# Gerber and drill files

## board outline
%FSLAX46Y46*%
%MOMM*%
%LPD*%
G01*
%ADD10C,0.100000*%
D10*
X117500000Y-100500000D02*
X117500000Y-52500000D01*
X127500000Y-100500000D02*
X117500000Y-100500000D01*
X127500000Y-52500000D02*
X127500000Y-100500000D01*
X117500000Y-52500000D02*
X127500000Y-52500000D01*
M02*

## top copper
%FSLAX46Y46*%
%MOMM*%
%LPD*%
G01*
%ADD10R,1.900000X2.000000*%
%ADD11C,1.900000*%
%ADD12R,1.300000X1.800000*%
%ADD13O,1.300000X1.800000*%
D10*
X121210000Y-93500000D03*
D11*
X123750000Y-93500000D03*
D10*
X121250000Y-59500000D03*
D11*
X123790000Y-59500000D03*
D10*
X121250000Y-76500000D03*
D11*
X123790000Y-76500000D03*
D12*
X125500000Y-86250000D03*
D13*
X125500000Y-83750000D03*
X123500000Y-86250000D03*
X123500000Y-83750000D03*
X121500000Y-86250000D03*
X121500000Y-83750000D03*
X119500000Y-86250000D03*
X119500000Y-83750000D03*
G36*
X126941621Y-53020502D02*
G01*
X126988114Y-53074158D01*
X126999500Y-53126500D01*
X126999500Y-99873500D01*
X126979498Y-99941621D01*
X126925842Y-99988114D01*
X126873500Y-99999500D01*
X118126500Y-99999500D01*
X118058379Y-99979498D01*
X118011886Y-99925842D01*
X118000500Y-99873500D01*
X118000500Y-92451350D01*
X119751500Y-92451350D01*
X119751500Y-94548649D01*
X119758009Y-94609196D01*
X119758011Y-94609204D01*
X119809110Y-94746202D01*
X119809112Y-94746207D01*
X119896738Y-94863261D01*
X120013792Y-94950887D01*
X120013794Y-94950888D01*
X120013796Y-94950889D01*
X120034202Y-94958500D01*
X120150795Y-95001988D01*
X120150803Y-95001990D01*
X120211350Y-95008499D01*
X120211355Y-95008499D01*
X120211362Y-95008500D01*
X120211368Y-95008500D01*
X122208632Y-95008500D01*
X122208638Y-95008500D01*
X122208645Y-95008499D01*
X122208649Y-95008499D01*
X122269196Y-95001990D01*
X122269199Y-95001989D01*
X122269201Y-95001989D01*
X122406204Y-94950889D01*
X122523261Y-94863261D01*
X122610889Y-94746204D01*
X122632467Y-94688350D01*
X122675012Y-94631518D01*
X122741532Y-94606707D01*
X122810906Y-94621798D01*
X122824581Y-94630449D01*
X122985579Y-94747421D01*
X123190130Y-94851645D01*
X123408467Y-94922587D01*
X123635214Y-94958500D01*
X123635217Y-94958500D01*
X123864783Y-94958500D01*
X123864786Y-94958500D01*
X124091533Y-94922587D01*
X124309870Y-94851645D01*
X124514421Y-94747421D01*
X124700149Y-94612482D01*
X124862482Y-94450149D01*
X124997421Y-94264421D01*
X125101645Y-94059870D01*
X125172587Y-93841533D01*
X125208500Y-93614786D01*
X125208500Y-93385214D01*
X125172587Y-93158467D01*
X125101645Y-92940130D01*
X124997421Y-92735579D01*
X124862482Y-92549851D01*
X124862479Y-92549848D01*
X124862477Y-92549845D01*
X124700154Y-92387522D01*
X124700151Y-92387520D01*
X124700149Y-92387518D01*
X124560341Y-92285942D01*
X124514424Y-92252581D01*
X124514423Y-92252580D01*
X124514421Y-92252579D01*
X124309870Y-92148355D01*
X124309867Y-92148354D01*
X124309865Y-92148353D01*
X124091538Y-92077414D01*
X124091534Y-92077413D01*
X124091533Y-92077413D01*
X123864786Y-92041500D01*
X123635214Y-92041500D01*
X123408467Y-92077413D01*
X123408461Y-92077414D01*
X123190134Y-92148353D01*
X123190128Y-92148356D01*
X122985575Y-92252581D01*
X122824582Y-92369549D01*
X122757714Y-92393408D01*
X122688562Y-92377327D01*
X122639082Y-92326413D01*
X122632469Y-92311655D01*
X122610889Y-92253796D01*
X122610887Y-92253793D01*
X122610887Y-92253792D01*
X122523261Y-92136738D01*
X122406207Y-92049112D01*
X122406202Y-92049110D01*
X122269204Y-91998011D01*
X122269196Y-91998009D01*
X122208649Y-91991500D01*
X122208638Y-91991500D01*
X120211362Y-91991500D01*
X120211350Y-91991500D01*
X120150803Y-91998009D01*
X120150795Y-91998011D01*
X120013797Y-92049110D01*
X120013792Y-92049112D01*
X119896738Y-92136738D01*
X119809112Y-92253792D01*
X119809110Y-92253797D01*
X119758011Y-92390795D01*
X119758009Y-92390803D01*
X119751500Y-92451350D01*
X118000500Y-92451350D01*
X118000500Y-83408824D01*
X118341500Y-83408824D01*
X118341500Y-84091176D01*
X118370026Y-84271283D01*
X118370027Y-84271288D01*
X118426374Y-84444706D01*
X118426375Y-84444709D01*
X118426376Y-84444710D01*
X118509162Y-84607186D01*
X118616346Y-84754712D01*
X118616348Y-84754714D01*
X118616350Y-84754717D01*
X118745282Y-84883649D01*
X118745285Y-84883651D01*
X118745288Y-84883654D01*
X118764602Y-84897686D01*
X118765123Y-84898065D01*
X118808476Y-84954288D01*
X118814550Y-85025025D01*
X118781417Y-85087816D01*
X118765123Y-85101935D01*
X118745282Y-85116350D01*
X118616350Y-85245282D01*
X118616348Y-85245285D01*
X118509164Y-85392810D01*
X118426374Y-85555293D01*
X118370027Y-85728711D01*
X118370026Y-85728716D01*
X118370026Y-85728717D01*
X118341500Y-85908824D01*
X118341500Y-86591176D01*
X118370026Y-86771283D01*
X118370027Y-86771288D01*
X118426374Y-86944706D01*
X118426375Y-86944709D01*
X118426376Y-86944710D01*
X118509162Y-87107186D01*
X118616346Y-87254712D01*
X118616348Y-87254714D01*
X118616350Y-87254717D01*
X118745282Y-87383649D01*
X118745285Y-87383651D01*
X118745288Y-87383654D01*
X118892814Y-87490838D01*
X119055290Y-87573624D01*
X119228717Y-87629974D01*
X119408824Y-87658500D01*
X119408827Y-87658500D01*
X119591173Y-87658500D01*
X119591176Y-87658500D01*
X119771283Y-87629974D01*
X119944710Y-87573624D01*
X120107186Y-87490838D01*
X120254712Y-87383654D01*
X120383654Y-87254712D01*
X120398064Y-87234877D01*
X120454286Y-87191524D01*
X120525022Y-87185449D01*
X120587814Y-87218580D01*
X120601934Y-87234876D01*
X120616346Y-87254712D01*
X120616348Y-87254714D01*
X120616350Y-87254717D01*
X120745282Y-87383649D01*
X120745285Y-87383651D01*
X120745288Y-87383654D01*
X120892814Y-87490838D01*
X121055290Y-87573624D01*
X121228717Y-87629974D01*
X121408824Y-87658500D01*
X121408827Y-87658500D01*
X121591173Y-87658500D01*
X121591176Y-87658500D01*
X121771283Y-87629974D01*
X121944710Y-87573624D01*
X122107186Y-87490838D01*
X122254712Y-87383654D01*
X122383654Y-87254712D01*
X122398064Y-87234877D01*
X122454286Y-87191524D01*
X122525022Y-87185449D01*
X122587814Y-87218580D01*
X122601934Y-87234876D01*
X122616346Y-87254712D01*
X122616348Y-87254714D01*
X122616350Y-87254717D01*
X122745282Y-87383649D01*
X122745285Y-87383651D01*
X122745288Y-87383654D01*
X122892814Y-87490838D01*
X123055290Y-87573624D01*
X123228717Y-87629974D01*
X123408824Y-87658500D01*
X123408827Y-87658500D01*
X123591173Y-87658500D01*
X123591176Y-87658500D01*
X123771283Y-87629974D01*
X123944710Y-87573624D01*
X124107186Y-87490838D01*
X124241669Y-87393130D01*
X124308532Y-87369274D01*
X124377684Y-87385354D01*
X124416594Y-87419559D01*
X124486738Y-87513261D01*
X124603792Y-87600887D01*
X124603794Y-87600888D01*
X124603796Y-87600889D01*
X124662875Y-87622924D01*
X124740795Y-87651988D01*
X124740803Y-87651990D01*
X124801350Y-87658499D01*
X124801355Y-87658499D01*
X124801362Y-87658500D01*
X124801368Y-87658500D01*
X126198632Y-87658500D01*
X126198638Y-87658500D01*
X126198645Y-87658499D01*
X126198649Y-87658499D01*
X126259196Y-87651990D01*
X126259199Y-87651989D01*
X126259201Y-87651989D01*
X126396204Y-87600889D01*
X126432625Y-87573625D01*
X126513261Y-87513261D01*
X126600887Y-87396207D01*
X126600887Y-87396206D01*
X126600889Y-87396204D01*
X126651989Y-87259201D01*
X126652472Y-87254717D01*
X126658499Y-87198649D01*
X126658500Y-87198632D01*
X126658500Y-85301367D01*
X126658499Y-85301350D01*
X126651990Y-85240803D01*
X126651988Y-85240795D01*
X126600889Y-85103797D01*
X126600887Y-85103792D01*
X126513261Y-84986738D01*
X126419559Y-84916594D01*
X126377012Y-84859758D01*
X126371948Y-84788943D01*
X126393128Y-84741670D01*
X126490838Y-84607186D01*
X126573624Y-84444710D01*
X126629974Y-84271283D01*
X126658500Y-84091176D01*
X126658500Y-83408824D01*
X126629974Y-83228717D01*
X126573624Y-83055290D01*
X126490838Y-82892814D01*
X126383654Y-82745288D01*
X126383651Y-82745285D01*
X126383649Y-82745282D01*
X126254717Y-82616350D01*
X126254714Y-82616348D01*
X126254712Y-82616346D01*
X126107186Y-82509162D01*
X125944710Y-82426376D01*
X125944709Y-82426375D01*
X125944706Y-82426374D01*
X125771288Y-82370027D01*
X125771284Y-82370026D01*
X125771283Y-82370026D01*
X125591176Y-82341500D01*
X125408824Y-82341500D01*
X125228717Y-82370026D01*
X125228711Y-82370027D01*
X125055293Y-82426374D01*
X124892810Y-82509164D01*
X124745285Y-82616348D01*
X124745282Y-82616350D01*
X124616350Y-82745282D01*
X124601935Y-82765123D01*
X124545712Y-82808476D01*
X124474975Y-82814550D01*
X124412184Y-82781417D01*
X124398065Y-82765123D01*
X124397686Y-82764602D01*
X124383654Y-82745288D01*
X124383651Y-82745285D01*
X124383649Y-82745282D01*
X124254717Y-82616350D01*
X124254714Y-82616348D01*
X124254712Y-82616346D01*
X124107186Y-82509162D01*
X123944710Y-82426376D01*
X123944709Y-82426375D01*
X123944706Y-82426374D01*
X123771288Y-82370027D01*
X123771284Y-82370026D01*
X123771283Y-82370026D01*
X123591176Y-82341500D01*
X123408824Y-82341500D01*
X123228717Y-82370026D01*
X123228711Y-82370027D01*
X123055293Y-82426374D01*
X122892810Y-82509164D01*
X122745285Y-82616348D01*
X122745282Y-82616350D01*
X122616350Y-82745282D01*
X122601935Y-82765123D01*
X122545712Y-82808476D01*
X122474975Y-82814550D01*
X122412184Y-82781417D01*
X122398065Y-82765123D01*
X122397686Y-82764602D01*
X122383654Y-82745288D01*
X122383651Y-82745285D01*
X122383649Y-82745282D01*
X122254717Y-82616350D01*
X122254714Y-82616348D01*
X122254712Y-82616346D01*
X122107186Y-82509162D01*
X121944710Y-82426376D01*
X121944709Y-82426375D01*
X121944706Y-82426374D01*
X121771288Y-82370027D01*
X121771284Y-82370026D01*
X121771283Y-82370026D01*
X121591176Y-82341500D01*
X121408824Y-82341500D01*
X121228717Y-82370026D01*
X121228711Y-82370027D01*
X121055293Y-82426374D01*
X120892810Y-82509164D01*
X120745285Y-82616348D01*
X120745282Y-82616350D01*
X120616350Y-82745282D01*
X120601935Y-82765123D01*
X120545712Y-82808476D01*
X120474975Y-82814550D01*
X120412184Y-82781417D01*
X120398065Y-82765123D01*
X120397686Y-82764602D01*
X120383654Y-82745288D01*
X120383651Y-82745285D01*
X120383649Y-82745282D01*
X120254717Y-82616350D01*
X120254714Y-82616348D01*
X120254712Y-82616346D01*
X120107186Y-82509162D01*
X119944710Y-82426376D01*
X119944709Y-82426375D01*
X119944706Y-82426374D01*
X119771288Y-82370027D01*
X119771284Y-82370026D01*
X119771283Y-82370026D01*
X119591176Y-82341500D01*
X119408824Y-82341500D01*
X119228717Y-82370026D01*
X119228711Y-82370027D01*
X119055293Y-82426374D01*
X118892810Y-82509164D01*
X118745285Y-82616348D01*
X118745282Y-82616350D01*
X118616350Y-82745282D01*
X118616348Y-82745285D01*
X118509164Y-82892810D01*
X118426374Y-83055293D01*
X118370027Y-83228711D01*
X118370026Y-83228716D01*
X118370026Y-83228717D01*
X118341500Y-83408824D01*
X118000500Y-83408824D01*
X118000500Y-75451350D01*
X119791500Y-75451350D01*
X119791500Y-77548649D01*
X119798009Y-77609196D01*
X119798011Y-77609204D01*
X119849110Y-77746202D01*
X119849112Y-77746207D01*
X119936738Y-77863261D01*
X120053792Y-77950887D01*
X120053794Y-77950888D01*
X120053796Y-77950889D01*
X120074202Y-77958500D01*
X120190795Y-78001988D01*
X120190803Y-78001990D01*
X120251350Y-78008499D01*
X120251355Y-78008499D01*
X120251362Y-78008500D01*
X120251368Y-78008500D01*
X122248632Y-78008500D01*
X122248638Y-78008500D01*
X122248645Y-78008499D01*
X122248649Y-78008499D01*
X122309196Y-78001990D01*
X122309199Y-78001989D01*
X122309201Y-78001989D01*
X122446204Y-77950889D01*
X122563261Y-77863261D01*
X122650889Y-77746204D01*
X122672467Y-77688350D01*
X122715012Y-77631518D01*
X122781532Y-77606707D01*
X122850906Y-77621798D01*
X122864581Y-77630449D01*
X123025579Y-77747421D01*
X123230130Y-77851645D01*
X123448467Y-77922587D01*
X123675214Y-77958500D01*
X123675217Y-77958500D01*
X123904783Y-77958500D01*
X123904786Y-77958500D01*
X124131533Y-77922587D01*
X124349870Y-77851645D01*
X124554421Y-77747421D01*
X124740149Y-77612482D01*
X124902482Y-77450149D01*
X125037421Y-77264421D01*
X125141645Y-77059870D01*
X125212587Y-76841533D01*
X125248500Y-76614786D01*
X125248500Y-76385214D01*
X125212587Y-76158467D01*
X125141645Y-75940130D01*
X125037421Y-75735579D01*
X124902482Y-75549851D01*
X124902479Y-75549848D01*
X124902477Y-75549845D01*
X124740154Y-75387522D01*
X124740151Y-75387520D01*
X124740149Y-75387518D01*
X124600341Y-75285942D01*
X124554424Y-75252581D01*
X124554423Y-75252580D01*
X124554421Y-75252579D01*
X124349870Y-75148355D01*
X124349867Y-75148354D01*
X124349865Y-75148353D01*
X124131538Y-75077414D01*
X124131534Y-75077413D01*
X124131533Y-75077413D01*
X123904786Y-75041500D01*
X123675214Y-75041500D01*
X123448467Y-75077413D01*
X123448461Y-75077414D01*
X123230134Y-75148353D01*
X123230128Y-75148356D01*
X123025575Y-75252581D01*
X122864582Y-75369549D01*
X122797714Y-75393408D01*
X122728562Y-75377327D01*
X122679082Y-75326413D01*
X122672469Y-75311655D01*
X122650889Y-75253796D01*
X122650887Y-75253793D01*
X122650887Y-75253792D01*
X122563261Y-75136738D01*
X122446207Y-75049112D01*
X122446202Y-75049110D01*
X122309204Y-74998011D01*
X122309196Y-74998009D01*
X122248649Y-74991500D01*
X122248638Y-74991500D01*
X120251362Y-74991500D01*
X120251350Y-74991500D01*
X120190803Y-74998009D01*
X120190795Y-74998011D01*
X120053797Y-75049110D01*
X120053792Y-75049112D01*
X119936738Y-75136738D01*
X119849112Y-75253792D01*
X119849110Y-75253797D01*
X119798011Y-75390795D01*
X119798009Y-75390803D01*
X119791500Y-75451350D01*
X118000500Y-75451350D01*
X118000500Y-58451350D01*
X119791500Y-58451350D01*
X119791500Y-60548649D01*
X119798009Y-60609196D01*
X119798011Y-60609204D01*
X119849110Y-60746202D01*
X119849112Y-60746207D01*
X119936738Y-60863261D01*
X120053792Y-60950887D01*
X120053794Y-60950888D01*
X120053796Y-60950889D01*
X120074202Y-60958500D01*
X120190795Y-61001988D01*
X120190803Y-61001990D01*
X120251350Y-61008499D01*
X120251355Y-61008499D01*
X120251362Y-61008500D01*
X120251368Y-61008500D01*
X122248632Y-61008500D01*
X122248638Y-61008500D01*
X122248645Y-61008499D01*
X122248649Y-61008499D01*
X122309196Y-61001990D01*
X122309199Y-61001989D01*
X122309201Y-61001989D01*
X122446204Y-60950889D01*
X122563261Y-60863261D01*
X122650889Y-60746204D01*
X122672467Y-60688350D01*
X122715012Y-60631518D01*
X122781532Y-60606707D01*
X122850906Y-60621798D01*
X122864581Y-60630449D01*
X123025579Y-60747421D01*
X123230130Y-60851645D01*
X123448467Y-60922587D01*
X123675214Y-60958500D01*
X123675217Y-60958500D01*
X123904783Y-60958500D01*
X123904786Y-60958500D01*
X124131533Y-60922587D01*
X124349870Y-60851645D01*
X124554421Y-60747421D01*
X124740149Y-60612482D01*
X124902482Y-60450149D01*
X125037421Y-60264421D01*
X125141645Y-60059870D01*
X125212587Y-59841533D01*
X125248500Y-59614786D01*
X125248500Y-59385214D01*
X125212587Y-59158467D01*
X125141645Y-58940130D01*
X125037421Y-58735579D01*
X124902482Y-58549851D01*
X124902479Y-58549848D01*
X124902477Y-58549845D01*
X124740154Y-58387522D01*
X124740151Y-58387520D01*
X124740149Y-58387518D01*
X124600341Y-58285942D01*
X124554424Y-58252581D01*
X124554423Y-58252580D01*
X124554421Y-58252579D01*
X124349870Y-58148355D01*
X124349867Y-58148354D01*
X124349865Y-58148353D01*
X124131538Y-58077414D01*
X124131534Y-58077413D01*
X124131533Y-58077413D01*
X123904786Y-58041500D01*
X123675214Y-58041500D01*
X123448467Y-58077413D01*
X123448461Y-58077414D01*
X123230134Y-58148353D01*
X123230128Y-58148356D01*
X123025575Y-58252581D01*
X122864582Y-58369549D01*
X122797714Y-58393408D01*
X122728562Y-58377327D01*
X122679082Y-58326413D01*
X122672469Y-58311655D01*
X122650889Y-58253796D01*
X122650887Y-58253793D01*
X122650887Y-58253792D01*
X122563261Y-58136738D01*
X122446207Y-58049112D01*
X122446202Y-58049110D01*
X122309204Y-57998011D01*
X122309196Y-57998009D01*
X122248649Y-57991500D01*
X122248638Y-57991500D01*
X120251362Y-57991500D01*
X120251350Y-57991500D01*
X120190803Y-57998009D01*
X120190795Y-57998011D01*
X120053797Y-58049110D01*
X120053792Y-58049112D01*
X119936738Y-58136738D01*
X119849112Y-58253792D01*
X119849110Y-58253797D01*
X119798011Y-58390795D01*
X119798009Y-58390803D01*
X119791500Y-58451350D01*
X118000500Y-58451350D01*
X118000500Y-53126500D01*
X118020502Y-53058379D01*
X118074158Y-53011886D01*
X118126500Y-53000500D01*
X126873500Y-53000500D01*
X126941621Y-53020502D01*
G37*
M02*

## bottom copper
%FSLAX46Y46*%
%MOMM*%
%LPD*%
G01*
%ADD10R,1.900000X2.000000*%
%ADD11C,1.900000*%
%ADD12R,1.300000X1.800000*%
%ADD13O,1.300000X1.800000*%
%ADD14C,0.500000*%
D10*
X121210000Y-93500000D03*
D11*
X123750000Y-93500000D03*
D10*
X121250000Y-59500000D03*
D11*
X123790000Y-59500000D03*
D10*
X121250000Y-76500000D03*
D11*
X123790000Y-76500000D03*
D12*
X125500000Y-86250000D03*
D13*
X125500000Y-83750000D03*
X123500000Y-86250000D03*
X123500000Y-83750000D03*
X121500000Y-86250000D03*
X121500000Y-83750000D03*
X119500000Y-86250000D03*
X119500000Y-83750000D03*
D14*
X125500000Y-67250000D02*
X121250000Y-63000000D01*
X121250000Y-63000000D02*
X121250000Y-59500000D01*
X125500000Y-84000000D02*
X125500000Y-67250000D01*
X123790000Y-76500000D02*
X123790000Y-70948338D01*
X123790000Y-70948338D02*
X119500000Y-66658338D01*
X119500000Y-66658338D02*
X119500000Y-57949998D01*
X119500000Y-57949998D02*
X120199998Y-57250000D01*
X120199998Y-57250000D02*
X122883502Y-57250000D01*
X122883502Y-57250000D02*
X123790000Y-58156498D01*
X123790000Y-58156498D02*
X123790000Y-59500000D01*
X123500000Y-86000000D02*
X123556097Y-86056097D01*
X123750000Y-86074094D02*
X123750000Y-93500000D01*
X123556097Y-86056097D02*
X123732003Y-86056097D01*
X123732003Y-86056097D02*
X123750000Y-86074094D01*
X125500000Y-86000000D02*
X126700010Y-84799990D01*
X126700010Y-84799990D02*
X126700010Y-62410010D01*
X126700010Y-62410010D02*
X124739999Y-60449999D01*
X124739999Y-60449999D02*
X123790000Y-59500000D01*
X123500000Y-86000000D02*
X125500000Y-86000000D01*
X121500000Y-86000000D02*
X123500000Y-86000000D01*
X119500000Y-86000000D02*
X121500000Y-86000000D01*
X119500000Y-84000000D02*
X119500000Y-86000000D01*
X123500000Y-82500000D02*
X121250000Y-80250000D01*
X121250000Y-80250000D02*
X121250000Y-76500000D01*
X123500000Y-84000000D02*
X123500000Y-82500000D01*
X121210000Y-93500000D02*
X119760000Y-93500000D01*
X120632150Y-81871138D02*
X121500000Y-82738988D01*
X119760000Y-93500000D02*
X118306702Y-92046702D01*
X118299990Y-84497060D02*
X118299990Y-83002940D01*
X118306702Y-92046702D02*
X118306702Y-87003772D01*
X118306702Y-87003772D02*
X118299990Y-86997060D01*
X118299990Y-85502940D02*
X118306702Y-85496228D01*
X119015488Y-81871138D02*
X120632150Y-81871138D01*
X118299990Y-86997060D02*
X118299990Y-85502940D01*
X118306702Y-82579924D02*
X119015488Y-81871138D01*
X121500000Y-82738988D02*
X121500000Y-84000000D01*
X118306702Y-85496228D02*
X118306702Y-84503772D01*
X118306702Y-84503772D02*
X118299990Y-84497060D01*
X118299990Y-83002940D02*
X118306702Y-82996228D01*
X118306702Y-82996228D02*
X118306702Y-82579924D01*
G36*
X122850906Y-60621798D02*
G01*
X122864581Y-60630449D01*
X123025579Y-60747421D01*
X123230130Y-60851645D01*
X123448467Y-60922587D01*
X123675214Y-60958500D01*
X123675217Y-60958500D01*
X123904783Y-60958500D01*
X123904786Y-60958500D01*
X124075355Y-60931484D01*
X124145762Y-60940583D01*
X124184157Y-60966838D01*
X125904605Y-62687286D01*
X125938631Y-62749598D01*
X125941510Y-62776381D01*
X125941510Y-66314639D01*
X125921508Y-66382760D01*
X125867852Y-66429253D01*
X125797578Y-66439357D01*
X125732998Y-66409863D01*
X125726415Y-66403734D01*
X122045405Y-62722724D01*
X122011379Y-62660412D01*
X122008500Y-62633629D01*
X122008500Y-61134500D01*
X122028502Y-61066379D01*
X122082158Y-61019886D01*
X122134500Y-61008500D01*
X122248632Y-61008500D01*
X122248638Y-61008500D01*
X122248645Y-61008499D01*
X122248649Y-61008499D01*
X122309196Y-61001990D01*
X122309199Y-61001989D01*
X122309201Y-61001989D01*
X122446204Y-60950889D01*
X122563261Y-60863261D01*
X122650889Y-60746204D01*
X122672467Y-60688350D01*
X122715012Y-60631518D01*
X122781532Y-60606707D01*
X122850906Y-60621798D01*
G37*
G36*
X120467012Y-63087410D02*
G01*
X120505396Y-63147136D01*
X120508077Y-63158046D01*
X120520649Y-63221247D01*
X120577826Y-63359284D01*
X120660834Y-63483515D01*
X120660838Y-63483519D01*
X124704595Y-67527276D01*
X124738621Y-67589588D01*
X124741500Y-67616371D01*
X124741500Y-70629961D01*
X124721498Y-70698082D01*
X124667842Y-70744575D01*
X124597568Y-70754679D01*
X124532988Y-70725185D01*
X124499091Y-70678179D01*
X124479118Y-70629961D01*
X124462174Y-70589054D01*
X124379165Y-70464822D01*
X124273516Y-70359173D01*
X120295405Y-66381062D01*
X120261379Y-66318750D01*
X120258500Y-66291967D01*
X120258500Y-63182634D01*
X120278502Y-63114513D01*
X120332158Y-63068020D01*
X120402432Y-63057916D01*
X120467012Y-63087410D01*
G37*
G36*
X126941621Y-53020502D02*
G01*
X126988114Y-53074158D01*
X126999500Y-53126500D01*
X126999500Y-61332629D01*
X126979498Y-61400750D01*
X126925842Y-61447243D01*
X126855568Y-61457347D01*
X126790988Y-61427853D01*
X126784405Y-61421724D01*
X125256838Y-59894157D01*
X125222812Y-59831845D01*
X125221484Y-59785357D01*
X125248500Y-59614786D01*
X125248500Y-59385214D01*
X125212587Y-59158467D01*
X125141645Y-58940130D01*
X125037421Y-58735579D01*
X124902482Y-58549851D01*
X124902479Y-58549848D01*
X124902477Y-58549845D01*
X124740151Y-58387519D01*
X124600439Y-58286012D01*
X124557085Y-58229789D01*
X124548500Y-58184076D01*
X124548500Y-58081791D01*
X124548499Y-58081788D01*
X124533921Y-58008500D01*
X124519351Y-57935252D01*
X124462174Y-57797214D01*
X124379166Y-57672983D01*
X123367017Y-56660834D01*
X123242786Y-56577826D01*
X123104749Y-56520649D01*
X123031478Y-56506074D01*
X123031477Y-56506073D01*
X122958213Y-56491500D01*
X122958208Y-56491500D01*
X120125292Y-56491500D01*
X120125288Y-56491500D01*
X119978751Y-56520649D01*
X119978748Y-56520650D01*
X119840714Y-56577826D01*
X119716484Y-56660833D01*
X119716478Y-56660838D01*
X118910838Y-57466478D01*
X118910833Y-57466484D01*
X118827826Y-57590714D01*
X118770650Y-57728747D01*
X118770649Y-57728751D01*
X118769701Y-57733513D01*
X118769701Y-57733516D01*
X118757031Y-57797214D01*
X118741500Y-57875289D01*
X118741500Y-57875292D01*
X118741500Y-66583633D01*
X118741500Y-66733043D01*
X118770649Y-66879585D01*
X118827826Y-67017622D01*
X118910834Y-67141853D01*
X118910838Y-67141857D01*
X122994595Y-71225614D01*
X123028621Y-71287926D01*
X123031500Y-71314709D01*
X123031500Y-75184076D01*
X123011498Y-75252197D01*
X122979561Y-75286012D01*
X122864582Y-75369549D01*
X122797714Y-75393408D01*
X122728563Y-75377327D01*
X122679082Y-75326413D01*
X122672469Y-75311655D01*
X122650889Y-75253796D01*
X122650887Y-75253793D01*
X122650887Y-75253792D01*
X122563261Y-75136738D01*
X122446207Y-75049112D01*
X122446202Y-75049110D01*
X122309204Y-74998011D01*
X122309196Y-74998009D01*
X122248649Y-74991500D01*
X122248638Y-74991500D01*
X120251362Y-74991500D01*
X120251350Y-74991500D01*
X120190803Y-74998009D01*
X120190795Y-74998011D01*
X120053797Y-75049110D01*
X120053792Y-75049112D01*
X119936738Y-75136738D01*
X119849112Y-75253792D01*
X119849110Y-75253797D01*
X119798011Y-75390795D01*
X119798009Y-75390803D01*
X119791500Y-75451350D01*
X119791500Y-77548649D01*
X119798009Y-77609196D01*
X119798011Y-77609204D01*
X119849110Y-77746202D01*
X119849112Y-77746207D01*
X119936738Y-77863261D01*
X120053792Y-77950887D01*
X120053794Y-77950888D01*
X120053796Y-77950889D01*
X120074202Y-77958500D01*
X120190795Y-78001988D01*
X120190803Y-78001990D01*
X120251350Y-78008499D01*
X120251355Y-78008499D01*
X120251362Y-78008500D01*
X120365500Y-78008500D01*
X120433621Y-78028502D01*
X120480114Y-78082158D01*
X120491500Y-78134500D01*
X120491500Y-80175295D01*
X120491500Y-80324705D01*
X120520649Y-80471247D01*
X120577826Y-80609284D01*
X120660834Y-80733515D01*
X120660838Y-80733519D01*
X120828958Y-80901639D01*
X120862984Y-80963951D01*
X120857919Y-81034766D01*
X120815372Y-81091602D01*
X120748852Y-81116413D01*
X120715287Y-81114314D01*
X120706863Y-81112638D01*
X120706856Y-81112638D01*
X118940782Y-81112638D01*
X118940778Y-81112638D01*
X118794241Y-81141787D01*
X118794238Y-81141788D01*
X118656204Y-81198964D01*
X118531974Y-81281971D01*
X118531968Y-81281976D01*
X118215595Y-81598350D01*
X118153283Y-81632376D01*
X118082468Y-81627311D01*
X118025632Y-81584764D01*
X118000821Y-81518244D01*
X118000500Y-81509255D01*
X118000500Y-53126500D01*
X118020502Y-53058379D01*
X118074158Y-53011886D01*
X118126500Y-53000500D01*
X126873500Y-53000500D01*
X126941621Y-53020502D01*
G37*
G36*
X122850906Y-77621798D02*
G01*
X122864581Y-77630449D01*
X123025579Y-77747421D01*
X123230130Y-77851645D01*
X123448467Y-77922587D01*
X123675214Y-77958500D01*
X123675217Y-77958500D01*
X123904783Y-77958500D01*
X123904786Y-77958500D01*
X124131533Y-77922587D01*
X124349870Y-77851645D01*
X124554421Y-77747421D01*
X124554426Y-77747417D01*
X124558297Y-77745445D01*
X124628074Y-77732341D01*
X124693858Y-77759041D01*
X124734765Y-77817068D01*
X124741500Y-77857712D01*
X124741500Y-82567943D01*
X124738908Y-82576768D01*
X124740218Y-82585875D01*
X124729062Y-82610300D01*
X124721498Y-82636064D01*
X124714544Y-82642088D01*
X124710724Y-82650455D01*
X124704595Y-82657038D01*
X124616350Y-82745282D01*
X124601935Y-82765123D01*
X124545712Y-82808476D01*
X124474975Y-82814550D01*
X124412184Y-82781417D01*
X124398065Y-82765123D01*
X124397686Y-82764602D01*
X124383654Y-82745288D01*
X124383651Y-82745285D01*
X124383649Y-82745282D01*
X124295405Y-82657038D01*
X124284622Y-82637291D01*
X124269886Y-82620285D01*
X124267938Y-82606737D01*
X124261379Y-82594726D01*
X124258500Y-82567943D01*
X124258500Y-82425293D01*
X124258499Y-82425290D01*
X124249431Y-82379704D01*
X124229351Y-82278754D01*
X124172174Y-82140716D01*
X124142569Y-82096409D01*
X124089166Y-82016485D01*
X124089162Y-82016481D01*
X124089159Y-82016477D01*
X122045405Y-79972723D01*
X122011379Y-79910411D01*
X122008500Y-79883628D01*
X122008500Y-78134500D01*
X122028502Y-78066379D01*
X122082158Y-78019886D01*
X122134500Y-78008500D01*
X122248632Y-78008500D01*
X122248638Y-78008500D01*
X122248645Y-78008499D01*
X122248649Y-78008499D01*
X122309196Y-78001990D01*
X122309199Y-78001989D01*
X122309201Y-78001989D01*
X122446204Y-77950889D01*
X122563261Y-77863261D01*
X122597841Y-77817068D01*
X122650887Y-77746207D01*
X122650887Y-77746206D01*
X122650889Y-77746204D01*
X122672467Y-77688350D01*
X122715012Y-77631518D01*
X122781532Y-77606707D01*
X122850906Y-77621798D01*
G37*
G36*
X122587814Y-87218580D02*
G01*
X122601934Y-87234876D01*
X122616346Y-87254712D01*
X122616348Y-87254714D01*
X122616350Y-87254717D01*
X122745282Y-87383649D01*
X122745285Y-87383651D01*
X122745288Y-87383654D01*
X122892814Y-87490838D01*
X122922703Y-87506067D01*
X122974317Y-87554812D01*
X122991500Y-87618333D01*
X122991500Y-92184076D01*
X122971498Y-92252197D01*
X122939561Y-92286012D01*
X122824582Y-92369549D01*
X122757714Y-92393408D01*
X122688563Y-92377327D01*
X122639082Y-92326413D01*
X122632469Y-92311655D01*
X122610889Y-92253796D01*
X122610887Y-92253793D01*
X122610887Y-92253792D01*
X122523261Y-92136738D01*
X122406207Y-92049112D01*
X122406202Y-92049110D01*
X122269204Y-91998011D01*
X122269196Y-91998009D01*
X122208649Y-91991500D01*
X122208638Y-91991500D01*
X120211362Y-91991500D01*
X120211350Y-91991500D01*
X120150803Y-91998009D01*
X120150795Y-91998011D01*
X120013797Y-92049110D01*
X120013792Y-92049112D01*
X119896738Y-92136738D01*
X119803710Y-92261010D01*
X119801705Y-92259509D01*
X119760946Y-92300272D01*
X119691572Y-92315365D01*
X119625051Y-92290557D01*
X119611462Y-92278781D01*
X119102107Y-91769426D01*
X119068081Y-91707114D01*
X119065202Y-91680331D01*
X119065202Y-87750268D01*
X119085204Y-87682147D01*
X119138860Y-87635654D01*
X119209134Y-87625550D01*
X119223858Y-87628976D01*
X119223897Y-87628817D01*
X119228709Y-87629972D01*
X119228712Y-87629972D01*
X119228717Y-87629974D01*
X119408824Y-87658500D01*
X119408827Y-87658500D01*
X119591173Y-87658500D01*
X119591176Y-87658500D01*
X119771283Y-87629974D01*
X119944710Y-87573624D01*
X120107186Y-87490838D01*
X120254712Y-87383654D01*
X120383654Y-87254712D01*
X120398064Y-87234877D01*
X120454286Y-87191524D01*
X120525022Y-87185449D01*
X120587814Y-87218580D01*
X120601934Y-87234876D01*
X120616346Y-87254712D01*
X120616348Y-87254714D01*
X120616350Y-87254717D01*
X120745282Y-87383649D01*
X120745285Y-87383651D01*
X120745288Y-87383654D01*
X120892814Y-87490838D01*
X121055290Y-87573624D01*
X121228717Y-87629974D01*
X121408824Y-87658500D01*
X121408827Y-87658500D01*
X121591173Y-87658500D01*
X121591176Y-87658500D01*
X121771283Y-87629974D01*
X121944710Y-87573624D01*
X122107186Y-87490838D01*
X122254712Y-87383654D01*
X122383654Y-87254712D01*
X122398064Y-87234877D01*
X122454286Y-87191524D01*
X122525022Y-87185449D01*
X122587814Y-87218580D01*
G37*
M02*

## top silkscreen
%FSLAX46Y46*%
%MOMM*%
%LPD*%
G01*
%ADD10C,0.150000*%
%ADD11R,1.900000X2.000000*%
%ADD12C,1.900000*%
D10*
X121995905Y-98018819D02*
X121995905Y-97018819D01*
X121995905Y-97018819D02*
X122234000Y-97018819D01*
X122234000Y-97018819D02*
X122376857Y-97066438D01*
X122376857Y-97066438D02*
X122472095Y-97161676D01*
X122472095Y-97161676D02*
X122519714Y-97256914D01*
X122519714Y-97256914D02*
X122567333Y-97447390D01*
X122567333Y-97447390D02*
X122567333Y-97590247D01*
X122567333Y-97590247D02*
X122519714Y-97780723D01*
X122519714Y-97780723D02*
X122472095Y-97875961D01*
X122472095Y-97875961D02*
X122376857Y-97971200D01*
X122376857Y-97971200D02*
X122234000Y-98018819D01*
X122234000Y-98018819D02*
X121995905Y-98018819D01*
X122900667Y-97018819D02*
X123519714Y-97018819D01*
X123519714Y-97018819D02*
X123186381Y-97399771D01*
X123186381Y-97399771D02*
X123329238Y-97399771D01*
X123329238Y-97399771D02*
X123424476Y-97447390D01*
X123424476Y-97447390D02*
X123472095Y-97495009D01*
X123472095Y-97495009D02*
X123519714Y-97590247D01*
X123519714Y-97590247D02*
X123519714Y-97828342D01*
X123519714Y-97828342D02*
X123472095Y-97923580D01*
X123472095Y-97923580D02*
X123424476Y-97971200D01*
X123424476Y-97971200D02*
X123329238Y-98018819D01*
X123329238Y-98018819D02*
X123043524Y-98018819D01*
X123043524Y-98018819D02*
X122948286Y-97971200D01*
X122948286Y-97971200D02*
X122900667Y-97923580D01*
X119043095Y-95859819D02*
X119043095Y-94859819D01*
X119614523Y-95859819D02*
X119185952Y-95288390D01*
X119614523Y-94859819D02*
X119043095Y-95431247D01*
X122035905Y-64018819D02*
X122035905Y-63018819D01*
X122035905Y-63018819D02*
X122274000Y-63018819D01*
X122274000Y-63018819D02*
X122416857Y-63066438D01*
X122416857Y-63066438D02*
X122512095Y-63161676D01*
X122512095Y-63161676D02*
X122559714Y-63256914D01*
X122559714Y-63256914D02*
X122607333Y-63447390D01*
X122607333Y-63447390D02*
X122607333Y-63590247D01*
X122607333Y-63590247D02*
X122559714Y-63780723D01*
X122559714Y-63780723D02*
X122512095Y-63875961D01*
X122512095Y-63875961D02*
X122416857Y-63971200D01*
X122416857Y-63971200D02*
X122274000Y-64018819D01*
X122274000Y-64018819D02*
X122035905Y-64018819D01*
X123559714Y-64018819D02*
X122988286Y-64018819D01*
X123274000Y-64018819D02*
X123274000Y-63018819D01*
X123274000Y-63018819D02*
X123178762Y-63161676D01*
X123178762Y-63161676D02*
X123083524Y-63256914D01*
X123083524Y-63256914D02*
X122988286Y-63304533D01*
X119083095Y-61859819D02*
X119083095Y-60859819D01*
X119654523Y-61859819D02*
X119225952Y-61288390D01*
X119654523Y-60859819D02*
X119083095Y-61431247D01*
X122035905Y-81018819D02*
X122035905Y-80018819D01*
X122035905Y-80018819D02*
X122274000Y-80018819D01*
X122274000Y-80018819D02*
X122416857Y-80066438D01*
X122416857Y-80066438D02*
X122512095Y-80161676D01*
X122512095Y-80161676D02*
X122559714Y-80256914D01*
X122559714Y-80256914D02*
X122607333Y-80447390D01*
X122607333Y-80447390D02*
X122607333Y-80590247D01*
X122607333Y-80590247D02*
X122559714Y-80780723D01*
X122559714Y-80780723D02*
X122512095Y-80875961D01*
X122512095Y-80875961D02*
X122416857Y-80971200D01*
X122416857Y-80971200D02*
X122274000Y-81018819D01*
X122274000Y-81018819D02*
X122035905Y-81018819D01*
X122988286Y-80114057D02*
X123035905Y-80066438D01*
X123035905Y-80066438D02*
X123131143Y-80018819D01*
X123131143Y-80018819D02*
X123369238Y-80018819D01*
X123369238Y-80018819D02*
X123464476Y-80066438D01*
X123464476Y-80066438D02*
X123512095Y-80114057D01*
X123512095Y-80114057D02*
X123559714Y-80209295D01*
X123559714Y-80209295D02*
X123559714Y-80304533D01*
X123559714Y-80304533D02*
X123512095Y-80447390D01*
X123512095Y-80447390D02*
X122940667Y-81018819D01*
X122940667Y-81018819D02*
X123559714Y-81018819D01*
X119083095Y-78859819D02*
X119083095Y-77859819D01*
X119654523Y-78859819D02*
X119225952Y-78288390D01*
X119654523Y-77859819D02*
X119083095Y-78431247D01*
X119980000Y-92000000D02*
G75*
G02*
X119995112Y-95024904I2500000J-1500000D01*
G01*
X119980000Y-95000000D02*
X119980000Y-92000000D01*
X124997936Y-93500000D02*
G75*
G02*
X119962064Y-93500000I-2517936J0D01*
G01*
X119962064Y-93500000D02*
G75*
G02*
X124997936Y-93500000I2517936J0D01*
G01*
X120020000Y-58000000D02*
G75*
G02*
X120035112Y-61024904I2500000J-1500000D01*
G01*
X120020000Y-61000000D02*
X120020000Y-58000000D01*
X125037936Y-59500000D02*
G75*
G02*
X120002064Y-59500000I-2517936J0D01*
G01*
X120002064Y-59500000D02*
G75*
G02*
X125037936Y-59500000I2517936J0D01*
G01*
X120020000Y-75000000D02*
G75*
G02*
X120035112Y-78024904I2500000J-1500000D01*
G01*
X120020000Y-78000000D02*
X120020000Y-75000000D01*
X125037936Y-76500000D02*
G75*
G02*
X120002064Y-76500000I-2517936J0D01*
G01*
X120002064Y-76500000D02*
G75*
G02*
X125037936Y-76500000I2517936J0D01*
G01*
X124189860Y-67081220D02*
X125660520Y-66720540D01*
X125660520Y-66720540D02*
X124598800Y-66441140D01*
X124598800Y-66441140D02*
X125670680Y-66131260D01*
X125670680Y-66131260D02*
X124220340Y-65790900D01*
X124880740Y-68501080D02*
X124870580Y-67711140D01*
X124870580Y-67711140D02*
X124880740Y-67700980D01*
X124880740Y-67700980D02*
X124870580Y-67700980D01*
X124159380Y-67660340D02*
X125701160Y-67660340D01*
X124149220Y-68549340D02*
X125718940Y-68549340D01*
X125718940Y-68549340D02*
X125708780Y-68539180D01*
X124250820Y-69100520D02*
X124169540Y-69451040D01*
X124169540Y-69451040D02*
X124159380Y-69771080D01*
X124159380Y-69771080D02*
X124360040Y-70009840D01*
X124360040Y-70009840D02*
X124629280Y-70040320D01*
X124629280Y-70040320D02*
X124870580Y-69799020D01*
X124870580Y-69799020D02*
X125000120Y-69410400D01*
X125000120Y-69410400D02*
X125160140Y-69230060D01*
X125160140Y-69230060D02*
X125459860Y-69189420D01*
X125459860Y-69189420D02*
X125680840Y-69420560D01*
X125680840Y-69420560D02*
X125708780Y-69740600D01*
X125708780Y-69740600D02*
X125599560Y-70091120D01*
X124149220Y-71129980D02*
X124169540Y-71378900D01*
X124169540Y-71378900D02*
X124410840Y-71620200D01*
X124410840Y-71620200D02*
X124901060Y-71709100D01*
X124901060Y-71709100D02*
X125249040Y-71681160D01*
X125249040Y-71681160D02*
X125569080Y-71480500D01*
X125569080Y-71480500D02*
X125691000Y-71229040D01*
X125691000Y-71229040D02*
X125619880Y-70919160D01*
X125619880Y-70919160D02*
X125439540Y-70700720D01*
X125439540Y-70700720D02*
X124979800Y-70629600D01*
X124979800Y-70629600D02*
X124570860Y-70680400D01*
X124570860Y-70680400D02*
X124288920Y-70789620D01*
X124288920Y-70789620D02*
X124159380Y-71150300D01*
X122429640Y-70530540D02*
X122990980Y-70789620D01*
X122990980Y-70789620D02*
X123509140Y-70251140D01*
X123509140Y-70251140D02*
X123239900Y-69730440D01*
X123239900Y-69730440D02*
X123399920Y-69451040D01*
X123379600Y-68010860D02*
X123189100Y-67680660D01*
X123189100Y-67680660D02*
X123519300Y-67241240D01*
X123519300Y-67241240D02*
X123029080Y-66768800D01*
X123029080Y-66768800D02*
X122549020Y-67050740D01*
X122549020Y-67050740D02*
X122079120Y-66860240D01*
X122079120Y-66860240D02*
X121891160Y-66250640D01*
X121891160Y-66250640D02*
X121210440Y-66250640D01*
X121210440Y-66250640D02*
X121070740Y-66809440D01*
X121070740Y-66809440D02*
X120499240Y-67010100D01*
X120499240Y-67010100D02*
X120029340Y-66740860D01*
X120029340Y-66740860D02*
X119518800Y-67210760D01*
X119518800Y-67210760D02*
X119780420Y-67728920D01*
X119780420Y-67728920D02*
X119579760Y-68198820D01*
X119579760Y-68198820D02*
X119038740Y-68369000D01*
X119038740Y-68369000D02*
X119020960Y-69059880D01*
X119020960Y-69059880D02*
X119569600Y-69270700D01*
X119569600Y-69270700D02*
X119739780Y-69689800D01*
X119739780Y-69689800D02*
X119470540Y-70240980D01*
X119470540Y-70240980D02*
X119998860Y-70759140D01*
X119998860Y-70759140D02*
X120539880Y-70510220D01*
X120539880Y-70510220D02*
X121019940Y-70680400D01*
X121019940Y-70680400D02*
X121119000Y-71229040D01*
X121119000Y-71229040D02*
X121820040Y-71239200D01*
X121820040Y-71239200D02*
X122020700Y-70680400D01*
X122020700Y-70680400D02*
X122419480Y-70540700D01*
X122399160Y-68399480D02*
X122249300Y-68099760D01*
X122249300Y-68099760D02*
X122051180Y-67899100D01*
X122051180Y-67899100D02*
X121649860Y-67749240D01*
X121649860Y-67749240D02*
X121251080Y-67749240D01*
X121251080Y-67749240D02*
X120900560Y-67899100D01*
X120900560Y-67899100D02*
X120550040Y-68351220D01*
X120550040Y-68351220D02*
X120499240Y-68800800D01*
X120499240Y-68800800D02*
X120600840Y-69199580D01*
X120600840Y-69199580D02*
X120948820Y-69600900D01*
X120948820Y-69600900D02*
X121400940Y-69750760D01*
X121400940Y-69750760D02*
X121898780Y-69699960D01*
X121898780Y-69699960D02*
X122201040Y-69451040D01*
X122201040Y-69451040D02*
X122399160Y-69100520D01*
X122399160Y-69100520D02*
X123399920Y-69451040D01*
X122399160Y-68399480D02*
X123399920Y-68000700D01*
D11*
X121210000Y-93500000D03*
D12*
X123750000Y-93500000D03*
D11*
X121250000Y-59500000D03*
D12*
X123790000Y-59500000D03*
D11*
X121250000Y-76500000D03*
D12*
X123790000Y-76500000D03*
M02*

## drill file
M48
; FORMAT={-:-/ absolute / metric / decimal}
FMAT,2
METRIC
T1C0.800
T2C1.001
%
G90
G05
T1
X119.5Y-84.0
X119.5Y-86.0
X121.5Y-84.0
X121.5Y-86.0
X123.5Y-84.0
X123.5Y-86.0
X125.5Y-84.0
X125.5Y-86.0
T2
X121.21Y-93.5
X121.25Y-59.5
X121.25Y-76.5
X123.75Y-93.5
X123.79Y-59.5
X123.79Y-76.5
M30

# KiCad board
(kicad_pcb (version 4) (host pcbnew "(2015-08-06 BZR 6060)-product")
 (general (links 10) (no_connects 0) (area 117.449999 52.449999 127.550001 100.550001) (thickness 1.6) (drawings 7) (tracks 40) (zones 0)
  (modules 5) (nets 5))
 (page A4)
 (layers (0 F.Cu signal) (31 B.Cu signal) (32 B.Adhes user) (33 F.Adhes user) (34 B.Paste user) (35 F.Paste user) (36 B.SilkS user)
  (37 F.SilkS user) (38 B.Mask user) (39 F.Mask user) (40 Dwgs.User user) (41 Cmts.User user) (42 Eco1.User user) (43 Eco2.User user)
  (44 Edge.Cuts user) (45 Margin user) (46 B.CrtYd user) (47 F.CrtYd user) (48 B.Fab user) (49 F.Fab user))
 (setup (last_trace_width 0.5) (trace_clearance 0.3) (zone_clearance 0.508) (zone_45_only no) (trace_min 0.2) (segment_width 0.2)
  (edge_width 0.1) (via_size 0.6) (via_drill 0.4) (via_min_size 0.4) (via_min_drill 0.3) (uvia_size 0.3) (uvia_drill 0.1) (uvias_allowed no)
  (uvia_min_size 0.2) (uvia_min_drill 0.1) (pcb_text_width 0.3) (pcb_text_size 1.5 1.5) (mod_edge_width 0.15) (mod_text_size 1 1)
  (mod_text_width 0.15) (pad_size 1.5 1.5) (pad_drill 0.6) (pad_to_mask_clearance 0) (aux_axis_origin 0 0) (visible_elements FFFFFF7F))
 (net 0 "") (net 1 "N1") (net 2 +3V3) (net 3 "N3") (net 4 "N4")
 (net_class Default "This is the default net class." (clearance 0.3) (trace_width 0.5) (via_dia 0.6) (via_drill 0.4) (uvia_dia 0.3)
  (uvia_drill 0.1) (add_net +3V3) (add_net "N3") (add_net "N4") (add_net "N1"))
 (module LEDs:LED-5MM (layer F.Cu) (at 121.21 93.5)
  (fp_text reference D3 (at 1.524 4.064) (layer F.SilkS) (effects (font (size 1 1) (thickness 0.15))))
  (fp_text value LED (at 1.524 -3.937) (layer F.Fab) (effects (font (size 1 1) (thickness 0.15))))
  (fp_arc (start 1.27 0) (end -1.23 -1.5) (angle 297.5) (layer F.SilkS) (width 0.15))
  (fp_line (start -1.23 1.5) (end -1.23 -1.5) (layer F.SilkS) (width 0.15))
  (fp_circle (center 1.27 0) (end 0.97 -2.5) (layer F.SilkS) (width 0.15))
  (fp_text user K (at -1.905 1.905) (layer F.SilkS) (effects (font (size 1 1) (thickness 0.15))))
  (pad 1 thru_hole rect (at 0 0 90) (size 2 1.9) (drill 1.00076) (layers *.Cu *.Mask F.SilkS) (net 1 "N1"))
  (pad 2 thru_hole circle (at 2.54 0) (size 1.9 1.9) (drill 1.00076) (layers *.Cu *.Mask F.SilkS) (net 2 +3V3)))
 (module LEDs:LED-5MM (layer F.Cu) (at 121.25 59.5)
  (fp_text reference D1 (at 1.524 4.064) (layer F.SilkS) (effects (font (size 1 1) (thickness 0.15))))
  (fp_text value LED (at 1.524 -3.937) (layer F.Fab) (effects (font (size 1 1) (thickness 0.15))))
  (fp_arc (start 1.27 0) (end -1.23 -1.5) (angle 297.5) (layer F.SilkS) (width 0.15))
  (fp_line (start -1.23 1.5) (end -1.23 -1.5) (layer F.SilkS) (width 0.15))
  (fp_circle (center 1.27 0) (end 0.97 -2.5) (layer F.SilkS) (width 0.15))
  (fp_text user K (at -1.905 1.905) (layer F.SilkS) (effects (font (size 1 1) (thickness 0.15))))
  (pad 1 thru_hole rect (at 0 0 90) (size 2 1.9) (drill 1.00076) (layers *.Cu *.Mask F.SilkS) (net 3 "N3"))
  (pad 2 thru_hole circle (at 2.54 0) (size 1.9 1.9) (drill 1.00076) (layers *.Cu *.Mask F.SilkS) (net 2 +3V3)))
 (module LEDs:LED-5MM (layer F.Cu) (at 121.25 76.5)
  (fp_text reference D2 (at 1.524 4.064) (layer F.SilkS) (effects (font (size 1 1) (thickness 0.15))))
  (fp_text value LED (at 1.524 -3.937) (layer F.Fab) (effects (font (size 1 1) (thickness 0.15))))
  (fp_arc (start 1.27 0) (end -1.23 -1.5) (angle 297.5) (layer F.SilkS) (width 0.15))
  (fp_line (start -1.23 1.5) (end -1.23 -1.5) (layer F.SilkS) (width 0.15))
  (fp_circle (center 1.27 0) (end 0.97 -2.5) (layer F.SilkS) (width 0.15))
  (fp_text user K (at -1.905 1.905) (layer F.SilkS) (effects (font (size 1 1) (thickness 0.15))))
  (pad 1 thru_hole rect (at 0 0 90) (size 2 1.9) (drill 1.00076) (layers *.Cu *.Mask F.SilkS) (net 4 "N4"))
  (pad 2 thru_hole circle (at 2.54 0) (size 1.9 1.9) (drill 1.00076) (layers *.Cu *.Mask F.SilkS) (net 2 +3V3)))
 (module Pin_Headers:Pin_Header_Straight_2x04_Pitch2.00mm (layer B.Cu) (at 122.5 85 180)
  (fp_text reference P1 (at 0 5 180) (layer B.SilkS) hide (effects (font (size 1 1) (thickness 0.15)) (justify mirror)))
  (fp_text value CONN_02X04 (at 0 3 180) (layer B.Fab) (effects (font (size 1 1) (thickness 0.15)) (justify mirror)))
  (pad 1 thru_hole rect (at -3 -1 180) (size 1.3 1.8) (drill 0.8 (offset 0 -0.25)) (layers *.Cu *.Mask B.SilkS) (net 2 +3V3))
  (pad 2 thru_hole oval (at -3 1 180) (size 1.3 1.8) (drill 0.8 (offset 0 0.25)) (layers *.Cu *.Mask B.SilkS) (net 3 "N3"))
  (pad 3 thru_hole oval (at -1 -1 180) (size 1.3 1.8) (drill 0.8 (offset 0 -0.25)) (layers *.Cu *.Mask B.SilkS) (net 2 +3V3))
  (pad 4 thru_hole oval (at -1 1 180) (size 1.3 1.8) (drill 0.8 (offset 0 0.25)) (layers *.Cu *.Mask B.SilkS) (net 4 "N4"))
  (pad 5 thru_hole oval (at 1 -1 180) (size 1.3 1.8) (drill 0.8 (offset 0 -0.25)) (layers *.Cu *.Mask B.SilkS) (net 2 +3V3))
  (pad 6 thru_hole oval (at 1 1 180) (size 1.3 1.8) (drill 0.8 (offset 0 0.25)) (layers *.Cu *.Mask B.SilkS) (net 1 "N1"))
  (pad 7 thru_hole oval (at 3 -1 180) (size 1.3 1.8) (drill 0.8 (offset 0 -0.25)) (layers *.Cu *.Mask B.SilkS) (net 2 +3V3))
  (pad 8 thru_hole oval (at 3 1 180) (size 1.3 1.8) (drill 0.8 (offset 0 0.25)) (layers *.Cu *.Mask B.SilkS) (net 2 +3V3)))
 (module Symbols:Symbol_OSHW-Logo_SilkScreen (layer F.Cu) (at 121.5 68.75 90)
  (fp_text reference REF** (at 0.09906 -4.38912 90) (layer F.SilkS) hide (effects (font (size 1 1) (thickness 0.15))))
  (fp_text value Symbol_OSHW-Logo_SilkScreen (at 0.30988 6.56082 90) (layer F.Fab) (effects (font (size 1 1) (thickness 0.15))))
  (fp_line (start 1.66878 2.68986) (end 2.02946 4.16052) (layer F.SilkS) (width 0.15))
  (fp_line (start 2.02946 4.16052) (end 2.30886 3.0988) (layer F.SilkS) (width 0.15))
  (fp_line (start 2.30886 3.0988) (end 2.61874 4.17068) (layer F.SilkS) (width 0.15))
  (fp_line (start 2.61874 4.17068) (end 2.9591 2.72034) (layer F.SilkS) (width 0.15))
  (fp_line (start 0.24892 3.38074) (end 1.03886 3.37058) (layer F.SilkS) (width 0.15))
  (fp_line (start 1.03886 3.37058) (end 1.04902 3.38074) (layer F.SilkS) (width 0.15))
  (fp_line (start 1.04902 3.38074) (end 1.04902 3.37058) (layer F.SilkS) (width 0.15))
  (fp_line (start 1.08966 2.65938) (end 1.08966 4.20116) (layer F.SilkS) (width 0.15))
  (fp_line (start 0.20066 2.64922) (end 0.20066 4.21894) (layer F.SilkS) (width 0.15))
  (fp_line (start 0.20066 4.21894) (end 0.21082 4.20878) (layer F.SilkS) (width 0.15))
  (fp_line (start -0.35052 2.75082) (end -0.70104 2.66954) (layer F.SilkS) (width 0.15))
  (fp_line (start -0.70104 2.66954) (end -1.02108 2.65938) (layer F.SilkS) (width 0.15))
  (fp_line (start -1.02108 2.65938) (end -1.25984 2.86004) (layer F.SilkS) (width 0.15))
  (fp_line (start -1.25984 2.86004) (end -1.29032 3.12928) (layer F.SilkS) (width 0.15))
  (fp_line (start -1.29032 3.12928) (end -1.04902 3.37058) (layer F.SilkS) (width 0.15))
  (fp_line (start -1.04902 3.37058) (end -0.6604 3.50012) (layer F.SilkS) (width 0.15))
  (fp_line (start -0.6604 3.50012) (end -0.48006 3.66014) (layer F.SilkS) (width 0.15))
  (fp_line (start -0.48006 3.66014) (end -0.43942 3.95986) (layer F.SilkS) (width 0.15))
  (fp_line (start -0.43942 3.95986) (end -0.67056 4.18084) (layer F.SilkS) (width 0.15))
  (fp_line (start -0.67056 4.18084) (end -0.9906 4.20878) (layer F.SilkS) (width 0.15))
  (fp_line (start -0.9906 4.20878) (end -1.34112 4.09956) (layer F.SilkS) (width 0.15))
  (fp_line (start -2.37998 2.64922) (end -2.6289 2.66954) (layer F.SilkS) (width 0.15))
  (fp_line (start -2.6289 2.66954) (end -2.8702 2.91084) (layer F.SilkS) (width 0.15))
  (fp_line (start -2.8702 2.91084) (end -2.9591 3.40106) (layer F.SilkS) (width 0.15))
  (fp_line (start -2.9591 3.40106) (end -2.93116 3.74904) (layer F.SilkS) (width 0.15))
  (fp_line (start -2.93116 3.74904) (end -2.7305 4.06908) (layer F.SilkS) (width 0.15))
  (fp_line (start -2.7305 4.06908) (end -2.47904 4.191) (layer F.SilkS) (width 0.15))
  (fp_line (start -2.47904 4.191) (end -2.16916 4.11988) (layer F.SilkS) (width 0.15))
  (fp_line (start -2.16916 4.11988) (end -1.95072 3.93954) (layer F.SilkS) (width 0.15))
  (fp_line (start -1.95072 3.93954) (end -1.8796 3.4798) (layer F.SilkS) (width 0.15))
  (fp_line (start -1.8796 3.4798) (end -1.9304 3.07086) (layer F.SilkS) (width 0.15))
  (fp_line (start -1.9304 3.07086) (end -2.03962 2.78892) (layer F.SilkS) (width 0.15))
  (fp_line (start -2.03962 2.78892) (end -2.4003 2.65938) (layer F.SilkS) (width 0.15))
  (fp_line (start -1.78054 0.92964) (end -2.03962 1.49098) (layer F.SilkS) (width 0.15))
  (fp_line (start -2.03962 1.49098) (end -1.50114 2.00914) (layer F.SilkS) (width 0.15))
  (fp_line (start -1.50114 2.00914) (end -0.98044 1.7399) (layer F.SilkS) (width 0.15))
  (fp_line (start -0.98044 1.7399) (end -0.70104 1.89992) (layer F.SilkS) (width 0.15))
  (fp_line (start 0.73914 1.8796) (end 1.06934 1.6891) (layer F.SilkS) (width 0.15))
  (fp_line (start 1.06934 1.6891) (end 1.50876 2.0193) (layer F.SilkS) (width 0.15))
  (fp_line (start 1.50876 2.0193) (end 1.9812 1.52908) (layer F.SilkS) (width 0.15))
  (fp_line (start 1.9812 1.52908) (end 1.69926 1.04902) (layer F.SilkS) (width 0.15))
  (fp_line (start 1.69926 1.04902) (end 1.88976 0.57912) (layer F.SilkS) (width 0.15))
  (fp_line (start 1.88976 0.57912) (end 2.49936 0.39116) (layer F.SilkS) (width 0.15))
  (fp_line (start 2.49936 0.39116) (end 2.49936 -0.28956) (layer F.SilkS) (width 0.15))
  (fp_line (start 2.49936 -0.28956) (end 1.94056 -0.42926) (layer F.SilkS) (width 0.15))
  (fp_line (start 1.94056 -0.42926) (end 1.7399 -1.00076) (layer F.SilkS) (width 0.15))
  (fp_line (start 1.7399 -1.00076) (end 2.00914 -1.47066) (layer F.SilkS) (width 0.15))
  (fp_line (start 2.00914 -1.47066) (end 1.53924 -1.9812) (layer F.SilkS) (width 0.15))
  (fp_line (start 1.53924 -1.9812) (end 1.02108 -1.71958) (layer F.SilkS) (width 0.15))
  (fp_line (start 1.02108 -1.71958) (end 0.55118 -1.92024) (layer F.SilkS) (width 0.15))
  (fp_line (start 0.55118 -1.92024) (end 0.381 -2.46126) (layer F.SilkS) (width 0.15))
  (fp_line (start 0.381 -2.46126) (end -0.30988 -2.47904) (layer F.SilkS) (width 0.15))
  (fp_line (start -0.30988 -2.47904) (end -0.5207 -1.9304) (layer F.SilkS) (width 0.15))
  (fp_line (start -0.5207 -1.9304) (end -0.9398 -1.76022) (layer F.SilkS) (width 0.15))
  (fp_line (start -0.9398 -1.76022) (end -1.49098 -2.02946) (layer F.SilkS) (width 0.15))
  (fp_line (start -1.49098 -2.02946) (end -2.00914 -1.50114) (layer F.SilkS) (width 0.15))
  (fp_line (start -2.00914 -1.50114) (end -1.76022 -0.96012) (layer F.SilkS) (width 0.15))
  (fp_line (start -1.76022 -0.96012) (end -1.9304 -0.48006) (layer F.SilkS) (width 0.15))
  (fp_line (start -1.9304 -0.48006) (end -2.47904 -0.381) (layer F.SilkS) (width 0.15))
  (fp_line (start -2.47904 -0.381) (end -2.4892 0.32004) (layer F.SilkS) (width 0.15))
  (fp_line (start -2.4892 0.32004) (end -1.9304 0.5207) (layer F.SilkS) (width 0.15))
  (fp_line (start -1.9304 0.5207) (end -1.7907 0.91948) (layer F.SilkS) (width 0.15))
  (fp_line (start 0.35052 0.89916) (end 0.65024 0.7493) (layer F.SilkS) (width 0.15))
  (fp_line (start 0.65024 0.7493) (end 0.8509 0.55118) (layer F.SilkS) (width 0.15))
  (fp_line (start 0.8509 0.55118) (end 1.00076 0.14986) (layer F.SilkS) (width 0.15))
  (fp_line (start 1.00076 0.14986) (end 1.00076 -0.24892) (layer F.SilkS) (width 0.15))
  (fp_line (start 1.00076 -0.24892) (end 0.8509 -0.59944) (layer F.SilkS) (width 0.15))
  (fp_line (start 0.8509 -0.59944) (end 0.39878 -0.94996) (layer F.SilkS) (width 0.15))
  (fp_line (start 0.39878 -0.94996) (end -0.0508 -1.00076) (layer F.SilkS) (width 0.15))
  (fp_line (start -0.0508 -1.00076) (end -0.44958 -0.89916) (layer F.SilkS) (width 0.15))
  (fp_line (start -0.44958 -0.89916) (end -0.8509 -0.55118) (layer F.SilkS) (width 0.15))
  (fp_line (start -0.8509 -0.55118) (end -1.00076 -0.09906) (layer F.SilkS) (width 0.15))
  (fp_line (start -1.00076 -0.09906) (end -0.94996 0.39878) (layer F.SilkS) (width 0.15))
  (fp_line (start -0.94996 0.39878) (end -0.70104 0.70104) (layer F.SilkS) (width 0.15))
  (fp_line (start -0.70104 0.70104) (end -0.35052 0.89916) (layer F.SilkS) (width 0.15))
  (fp_line (start -0.35052 0.89916) (end -0.70104 1.89992) (layer F.SilkS) (width 0.15))
  (fp_line (start 0.35052 0.89916) (end 0.7493 1.89992) (layer F.SilkS) (width 0.15)))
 (gr_line (start 117.5 100.5) (end 117.5 52.5) (layer Edge.Cuts) (width 0.1))
 (gr_line (start 127.5 100.5) (end 117.5 100.5) (layer Edge.Cuts) (width 0.1))
 (gr_line (start 127.5 52.5) (end 127.5 100.5) (layer Edge.Cuts) (width 0.1))
 (gr_line (start 117.5 52.5) (end 127.5 52.5) (layer Edge.Cuts) (width 0.1))
 (segment (start 125.5 67.25) (end 121.25 63) (width 0.5) (layer B.Cu) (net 3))
 (segment (start 121.25 63) (end 121.25 59.5) (width 0.5) (layer B.Cu) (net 3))
 (segment (start 125.5 84) (end 125.5 67.25) (width 0.5) (layer B.Cu) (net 3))
 (segment (start 123.79 76.5) (end 123.79 70.948338) (width 0.5) (layer B.Cu) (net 2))
 (segment (start 123.79 70.948338) (end 119.5 66.658338) (width 0.5) (layer B.Cu) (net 2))
 (segment (start 119.5 66.658338) (end 119.5 57.949998) (width 0.5) (layer B.Cu) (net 2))
 (segment (start 119.5 57.949998) (end 120.199998 57.25) (width 0.5) (layer B.Cu) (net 2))
 (segment (start 120.199998 57.25) (end 122.883502 57.25) (width 0.5) (layer B.Cu) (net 2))
 (segment (start 122.883502 57.25) (end 123.79 58.156498) (width 0.5) (layer B.Cu) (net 2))
 (segment (start 123.79 58.156498) (end 123.79 59.5) (width 0.5) (layer B.Cu) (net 2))
 (segment (start 123.5 86) (end 123.556097 86.056097) (width 0.5) (layer B.Cu) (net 2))
 (segment (start 123.75 86.074094) (end 123.75 93.5) (width 0.5) (layer B.Cu) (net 2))
 (segment (start 123.556097 86.056097) (end 123.732003 86.056097) (width 0.5) (layer B.Cu) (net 2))
 (segment (start 123.732003 86.056097) (end 123.75 86.074094) (width 0.5) (layer B.Cu) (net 2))
 (segment (start 125.5 86) (end 126.70001 84.79999) (width 0.5) (layer B.Cu) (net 2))
 (segment (start 126.70001 84.79999) (end 126.70001 62.41001) (width 0.5) (layer B.Cu) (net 2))
 (segment (start 126.70001 62.41001) (end 124.739999 60.449999) (width 0.5) (layer B.Cu) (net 2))
 (segment (start 124.739999 60.449999) (end 123.79 59.5) (width 0.5) (layer B.Cu) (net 2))
 (segment (start 123.5 86) (end 125.5 86) (width 0.5) (layer B.Cu) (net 2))
 (segment (start 121.5 86) (end 123.5 86) (width 0.5) (layer B.Cu) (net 2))
 (segment (start 119.5 86) (end 121.5 86) (width 0.5) (layer B.Cu) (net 2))
 (segment (start 119.5 84) (end 119.5 86) (width 0.5) (layer B.Cu) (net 2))
 (segment (start 123.5 82.5) (end 121.25 80.25) (width 0.5) (layer B.Cu) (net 4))
 (segment (start 121.25 80.25) (end 121.25 76.5) (width 0.5) (layer B.Cu) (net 4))
 (segment (start 123.5 84) (end 123.5 82.5) (width 0.5) (layer B.Cu) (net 4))
 (segment (start 121.21 93.5) (end 119.76 93.5) (width 0.5) (layer B.Cu) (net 1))
 (segment (start 120.63215 81.871138) (end 121.5 82.738988) (width 0.5) (layer B.Cu) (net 1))
 (segment (start 119.76 93.5) (end 118.306702 92.046702) (width 0.5) (layer B.Cu) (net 1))
 (segment (start 118.29999 84.49706) (end 118.29999 83.00294) (width 0.5) (layer B.Cu) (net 1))
 (segment (start 118.306702 92.046702) (end 118.306702 87.003772) (width 0.5) (layer B.Cu) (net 1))
 (segment (start 118.306702 87.003772) (end 118.29999 86.99706) (width 0.5) (layer B.Cu) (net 1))
 (segment (start 118.29999 85.50294) (end 118.306702 85.496228) (width 0.5) (layer B.Cu) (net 1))
 (segment (start 119.015488 81.871138) (end 120.63215 81.871138) (width 0.5) (layer B.Cu) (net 1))
 (segment (start 118.29999 86.99706) (end 118.29999 85.50294) (width 0.5) (layer B.Cu) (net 1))
 (segment (start 118.306702 82.579924) (end 119.015488 81.871138) (width 0.5) (layer B.Cu) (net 1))
 (segment (start 121.5 82.738988) (end 121.5 84) (width 0.5) (layer B.Cu) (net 1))
 (segment (start 118.306702 85.496228) (end 118.306702 84.503772) (width 0.5) (layer B.Cu) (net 1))
 (segment (start 118.306702 84.503772) (end 118.29999 84.49706) (width 0.5) (layer B.Cu) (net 1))
 (segment (start 118.29999 83.00294) (end 118.306702 82.996228) (width 0.5) (layer B.Cu) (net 1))
 (segment (start 118.306702 82.996228) (end 118.306702 82.579924) (width 0.5) (layer B.Cu) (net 1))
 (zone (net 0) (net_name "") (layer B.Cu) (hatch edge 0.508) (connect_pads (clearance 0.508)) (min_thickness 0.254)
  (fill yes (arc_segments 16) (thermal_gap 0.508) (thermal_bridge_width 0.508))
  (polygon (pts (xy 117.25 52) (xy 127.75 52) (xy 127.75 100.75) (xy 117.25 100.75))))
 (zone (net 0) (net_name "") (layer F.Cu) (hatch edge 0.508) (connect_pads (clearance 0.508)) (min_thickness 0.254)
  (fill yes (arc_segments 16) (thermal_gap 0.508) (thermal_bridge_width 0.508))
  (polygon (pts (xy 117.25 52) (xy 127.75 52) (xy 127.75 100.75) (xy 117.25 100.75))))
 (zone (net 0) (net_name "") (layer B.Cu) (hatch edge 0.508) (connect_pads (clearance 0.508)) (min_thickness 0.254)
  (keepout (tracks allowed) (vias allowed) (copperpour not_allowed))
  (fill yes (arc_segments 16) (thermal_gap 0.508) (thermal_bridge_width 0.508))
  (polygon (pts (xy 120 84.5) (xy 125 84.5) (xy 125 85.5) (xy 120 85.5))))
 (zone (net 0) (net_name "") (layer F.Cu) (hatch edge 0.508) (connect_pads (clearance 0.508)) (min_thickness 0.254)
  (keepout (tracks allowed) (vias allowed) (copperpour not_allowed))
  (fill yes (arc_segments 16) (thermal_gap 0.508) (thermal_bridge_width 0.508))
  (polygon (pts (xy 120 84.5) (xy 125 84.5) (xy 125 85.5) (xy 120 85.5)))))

